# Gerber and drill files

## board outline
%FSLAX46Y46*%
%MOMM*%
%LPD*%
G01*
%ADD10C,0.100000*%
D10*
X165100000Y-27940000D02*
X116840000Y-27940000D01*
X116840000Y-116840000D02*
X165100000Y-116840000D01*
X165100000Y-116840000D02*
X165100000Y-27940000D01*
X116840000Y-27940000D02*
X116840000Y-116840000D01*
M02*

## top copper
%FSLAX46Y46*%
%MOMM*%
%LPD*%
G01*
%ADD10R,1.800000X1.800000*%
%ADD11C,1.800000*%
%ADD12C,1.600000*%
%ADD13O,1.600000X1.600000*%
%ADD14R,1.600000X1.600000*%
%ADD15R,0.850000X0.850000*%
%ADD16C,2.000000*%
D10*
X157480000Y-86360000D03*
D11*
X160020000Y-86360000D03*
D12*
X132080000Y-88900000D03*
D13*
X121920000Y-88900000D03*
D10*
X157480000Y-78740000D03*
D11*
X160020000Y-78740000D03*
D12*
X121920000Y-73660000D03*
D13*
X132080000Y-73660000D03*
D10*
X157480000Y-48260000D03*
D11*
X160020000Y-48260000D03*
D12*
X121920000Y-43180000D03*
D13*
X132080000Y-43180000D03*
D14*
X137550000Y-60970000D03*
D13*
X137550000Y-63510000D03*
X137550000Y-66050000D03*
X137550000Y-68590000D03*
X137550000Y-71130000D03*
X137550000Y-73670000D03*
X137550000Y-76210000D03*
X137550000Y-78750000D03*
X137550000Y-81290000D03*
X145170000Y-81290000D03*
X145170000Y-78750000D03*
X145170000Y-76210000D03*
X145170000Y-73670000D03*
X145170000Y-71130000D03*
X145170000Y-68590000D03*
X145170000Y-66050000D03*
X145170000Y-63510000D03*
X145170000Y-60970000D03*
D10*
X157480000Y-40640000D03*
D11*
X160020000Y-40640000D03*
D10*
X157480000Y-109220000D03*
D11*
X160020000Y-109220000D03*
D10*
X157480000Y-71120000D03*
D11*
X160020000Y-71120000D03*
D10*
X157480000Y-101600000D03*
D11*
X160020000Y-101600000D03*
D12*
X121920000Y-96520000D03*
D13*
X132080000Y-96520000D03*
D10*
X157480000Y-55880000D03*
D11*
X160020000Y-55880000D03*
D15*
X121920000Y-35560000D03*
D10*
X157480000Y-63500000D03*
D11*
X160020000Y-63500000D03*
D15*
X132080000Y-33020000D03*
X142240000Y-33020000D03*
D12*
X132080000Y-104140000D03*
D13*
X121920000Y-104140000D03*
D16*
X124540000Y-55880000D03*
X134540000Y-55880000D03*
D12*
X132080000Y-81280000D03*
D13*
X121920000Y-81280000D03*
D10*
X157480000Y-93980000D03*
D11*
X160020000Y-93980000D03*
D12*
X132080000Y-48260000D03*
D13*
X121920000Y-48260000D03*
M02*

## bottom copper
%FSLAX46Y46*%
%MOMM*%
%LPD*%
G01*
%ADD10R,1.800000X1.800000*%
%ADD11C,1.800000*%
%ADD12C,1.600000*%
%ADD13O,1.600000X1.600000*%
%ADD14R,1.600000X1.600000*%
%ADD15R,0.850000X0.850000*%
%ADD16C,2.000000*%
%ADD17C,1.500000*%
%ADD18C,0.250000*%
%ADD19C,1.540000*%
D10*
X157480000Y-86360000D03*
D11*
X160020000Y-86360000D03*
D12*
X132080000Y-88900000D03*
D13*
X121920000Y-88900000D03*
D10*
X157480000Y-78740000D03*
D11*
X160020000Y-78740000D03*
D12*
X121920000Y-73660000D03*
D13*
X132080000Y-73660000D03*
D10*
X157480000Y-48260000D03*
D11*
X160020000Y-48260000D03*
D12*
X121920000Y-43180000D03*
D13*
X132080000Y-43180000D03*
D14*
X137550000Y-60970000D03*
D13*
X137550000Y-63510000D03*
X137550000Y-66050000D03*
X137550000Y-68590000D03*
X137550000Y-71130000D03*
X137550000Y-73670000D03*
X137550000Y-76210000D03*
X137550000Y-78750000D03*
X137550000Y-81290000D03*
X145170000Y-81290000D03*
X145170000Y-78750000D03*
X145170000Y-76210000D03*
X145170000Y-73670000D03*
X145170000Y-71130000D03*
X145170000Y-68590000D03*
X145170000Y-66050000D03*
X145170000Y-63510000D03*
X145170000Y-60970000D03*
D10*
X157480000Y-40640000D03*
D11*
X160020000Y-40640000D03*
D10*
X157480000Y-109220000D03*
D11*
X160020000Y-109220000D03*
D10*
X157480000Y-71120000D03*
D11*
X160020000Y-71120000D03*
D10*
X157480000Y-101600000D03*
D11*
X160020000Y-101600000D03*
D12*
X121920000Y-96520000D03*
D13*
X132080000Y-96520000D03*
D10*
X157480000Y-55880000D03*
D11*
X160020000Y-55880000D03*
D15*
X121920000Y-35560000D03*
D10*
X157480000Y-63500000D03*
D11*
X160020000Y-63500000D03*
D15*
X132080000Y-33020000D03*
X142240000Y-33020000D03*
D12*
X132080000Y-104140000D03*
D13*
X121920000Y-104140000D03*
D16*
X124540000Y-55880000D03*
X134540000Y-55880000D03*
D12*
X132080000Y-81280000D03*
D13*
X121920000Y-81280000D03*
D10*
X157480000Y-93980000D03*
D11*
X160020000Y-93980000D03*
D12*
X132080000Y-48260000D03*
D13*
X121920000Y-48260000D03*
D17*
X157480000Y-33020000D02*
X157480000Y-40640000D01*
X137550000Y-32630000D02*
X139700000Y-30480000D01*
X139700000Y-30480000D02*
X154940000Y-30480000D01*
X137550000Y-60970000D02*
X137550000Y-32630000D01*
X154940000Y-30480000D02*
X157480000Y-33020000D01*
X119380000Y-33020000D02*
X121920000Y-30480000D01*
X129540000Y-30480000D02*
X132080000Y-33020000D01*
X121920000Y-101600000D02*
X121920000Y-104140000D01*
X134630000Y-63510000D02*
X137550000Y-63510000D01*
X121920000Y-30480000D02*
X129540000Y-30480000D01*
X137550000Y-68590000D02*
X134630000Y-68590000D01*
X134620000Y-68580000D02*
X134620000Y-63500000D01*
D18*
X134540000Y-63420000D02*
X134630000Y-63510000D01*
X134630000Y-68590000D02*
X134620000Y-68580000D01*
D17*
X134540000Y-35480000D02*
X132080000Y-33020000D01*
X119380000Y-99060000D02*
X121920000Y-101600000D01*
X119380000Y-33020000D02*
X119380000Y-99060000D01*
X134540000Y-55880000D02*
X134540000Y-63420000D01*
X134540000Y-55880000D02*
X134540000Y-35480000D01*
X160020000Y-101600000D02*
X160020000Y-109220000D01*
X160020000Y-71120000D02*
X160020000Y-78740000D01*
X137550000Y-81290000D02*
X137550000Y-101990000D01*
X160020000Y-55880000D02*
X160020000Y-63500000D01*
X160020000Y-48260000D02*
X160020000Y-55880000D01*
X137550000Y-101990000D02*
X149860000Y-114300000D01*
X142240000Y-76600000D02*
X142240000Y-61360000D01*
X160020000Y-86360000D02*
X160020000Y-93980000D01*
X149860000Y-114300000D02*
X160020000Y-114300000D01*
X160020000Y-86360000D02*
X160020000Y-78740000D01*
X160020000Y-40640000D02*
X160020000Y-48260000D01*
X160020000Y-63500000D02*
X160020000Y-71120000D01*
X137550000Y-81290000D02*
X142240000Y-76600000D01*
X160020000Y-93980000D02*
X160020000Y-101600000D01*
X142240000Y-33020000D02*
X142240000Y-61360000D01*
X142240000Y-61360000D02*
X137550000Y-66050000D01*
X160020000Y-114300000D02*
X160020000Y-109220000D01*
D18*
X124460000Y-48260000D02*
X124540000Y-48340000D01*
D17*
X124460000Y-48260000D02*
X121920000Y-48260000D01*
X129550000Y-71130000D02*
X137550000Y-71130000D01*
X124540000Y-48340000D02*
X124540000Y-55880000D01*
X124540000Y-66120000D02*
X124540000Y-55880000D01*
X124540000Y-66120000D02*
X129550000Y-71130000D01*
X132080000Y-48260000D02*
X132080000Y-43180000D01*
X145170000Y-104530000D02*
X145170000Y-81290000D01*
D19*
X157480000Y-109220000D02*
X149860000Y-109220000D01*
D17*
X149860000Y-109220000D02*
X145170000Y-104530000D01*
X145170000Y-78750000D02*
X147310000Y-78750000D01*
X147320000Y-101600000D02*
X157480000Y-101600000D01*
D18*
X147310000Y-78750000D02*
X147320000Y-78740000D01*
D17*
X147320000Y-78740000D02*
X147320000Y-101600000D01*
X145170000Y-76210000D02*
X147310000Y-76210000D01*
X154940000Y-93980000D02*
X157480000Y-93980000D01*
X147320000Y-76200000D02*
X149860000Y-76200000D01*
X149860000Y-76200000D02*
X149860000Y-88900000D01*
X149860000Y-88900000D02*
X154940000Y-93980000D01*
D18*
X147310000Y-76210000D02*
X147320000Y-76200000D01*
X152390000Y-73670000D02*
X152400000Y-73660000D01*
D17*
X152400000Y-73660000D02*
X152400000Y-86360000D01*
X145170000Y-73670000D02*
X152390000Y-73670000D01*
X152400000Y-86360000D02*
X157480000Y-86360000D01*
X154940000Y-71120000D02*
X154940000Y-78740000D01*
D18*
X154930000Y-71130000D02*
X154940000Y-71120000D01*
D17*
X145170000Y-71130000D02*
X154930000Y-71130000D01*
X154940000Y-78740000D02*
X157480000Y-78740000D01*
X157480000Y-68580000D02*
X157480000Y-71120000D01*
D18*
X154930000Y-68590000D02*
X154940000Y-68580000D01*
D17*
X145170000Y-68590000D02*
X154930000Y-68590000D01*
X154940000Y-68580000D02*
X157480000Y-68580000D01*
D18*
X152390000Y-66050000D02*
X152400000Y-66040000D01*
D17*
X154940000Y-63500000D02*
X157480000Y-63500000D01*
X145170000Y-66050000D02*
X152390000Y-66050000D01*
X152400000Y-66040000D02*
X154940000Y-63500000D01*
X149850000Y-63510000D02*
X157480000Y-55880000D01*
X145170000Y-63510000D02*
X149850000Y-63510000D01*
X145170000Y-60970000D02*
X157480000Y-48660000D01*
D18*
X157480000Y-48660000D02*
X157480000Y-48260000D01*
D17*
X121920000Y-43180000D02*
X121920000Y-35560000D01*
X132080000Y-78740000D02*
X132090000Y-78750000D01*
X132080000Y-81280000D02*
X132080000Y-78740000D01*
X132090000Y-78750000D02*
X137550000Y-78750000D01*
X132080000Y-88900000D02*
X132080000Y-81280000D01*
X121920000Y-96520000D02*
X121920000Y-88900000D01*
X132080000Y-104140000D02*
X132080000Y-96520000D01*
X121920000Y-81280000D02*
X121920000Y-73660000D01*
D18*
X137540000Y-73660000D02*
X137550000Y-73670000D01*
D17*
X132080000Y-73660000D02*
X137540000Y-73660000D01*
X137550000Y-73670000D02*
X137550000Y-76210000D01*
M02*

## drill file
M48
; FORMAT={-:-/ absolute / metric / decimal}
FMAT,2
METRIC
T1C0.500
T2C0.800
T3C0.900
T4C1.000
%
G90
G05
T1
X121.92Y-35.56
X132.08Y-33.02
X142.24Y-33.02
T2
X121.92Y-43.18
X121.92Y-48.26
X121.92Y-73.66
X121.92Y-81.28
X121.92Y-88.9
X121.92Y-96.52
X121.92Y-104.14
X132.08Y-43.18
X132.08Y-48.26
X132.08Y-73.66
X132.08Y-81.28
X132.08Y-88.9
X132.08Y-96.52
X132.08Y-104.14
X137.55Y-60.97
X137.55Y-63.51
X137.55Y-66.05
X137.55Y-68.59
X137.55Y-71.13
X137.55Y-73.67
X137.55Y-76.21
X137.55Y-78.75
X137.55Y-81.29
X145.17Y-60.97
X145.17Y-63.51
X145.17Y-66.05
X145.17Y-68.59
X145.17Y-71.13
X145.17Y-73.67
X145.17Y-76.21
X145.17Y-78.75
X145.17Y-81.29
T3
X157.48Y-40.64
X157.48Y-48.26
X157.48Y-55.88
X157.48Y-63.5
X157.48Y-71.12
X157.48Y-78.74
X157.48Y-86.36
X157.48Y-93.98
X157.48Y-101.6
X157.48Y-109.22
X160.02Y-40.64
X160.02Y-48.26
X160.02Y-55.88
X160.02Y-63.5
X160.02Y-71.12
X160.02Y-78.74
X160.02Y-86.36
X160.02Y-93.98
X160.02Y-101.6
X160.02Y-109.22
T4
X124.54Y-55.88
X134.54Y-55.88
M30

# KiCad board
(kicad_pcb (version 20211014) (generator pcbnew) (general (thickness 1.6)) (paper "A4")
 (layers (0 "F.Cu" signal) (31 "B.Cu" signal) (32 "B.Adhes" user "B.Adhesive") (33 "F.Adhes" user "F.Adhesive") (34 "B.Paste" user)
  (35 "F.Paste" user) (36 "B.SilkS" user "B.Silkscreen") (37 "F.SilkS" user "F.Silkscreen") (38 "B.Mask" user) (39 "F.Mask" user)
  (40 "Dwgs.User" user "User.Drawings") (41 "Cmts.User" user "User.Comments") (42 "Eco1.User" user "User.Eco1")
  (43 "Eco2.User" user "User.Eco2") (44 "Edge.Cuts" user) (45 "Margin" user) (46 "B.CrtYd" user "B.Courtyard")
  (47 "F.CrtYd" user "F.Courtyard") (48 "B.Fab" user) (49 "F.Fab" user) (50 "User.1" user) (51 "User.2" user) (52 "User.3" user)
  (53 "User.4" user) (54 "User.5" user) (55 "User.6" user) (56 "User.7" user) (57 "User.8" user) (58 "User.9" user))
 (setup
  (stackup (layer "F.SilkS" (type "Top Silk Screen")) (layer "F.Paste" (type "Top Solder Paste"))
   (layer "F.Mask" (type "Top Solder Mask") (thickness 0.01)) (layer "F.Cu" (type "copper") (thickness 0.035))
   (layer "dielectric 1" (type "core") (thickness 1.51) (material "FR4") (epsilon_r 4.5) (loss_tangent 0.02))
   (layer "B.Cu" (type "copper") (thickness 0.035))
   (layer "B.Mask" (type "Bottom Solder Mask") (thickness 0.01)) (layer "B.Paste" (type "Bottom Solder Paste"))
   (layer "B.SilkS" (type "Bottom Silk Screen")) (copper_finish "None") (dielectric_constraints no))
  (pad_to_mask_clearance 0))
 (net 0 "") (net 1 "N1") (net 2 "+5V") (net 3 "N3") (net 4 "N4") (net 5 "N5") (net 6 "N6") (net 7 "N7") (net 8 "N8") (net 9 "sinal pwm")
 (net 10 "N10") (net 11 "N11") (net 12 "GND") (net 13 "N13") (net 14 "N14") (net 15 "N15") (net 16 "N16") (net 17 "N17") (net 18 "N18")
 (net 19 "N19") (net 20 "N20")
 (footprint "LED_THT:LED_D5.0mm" (layer "F.Cu") (at 157.48 86.36)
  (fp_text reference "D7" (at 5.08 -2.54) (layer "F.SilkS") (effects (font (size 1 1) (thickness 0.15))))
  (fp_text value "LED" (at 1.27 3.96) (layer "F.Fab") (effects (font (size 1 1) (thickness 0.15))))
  (pad "1" thru_hole rect (at 0 0) (size 1.8 1.8) (drill 0.9) (layers *.Cu *.Mask) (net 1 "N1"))
  (pad "2" thru_hole circle (at 2.54 0) (size 1.8 1.8) (drill 0.9) (layers *.Cu *.Mask) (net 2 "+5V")))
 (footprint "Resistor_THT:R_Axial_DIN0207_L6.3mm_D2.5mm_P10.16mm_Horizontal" (layer "F.Cu") (at 132.08 88.9 180)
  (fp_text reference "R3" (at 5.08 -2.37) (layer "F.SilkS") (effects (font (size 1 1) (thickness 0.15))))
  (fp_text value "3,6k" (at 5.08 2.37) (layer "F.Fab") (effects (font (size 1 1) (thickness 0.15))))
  (pad "1" thru_hole circle (at 0 0 180) (size 1.6 1.6) (drill 0.8) (layers *.Cu *.Mask) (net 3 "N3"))
  (pad "2" thru_hole oval (at 10.16 0 180) (size 1.6 1.6) (drill 0.8) (layers *.Cu *.Mask) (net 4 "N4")))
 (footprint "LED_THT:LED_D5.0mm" (layer "F.Cu") (at 157.48 78.74)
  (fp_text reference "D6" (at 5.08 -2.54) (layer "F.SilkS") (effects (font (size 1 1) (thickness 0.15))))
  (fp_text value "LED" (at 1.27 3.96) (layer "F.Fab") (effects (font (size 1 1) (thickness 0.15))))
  (pad "1" thru_hole rect (at 0 0) (size 1.8 1.8) (drill 0.9) (layers *.Cu *.Mask) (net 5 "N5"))
  (pad "2" thru_hole circle (at 2.54 0) (size 1.8 1.8) (drill 0.9) (layers *.Cu *.Mask) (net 2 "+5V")))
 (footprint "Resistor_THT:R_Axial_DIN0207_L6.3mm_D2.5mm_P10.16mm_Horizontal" (layer "F.Cu") (at 121.92 73.66)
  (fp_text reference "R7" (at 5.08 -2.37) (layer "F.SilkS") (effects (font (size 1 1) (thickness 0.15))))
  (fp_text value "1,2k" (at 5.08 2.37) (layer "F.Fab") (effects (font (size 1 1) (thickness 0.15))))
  (pad "1" thru_hole circle (at 0 0) (size 1.6 1.6) (drill 0.8) (layers *.Cu *.Mask) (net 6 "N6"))
  (pad "2" thru_hole oval (at 10.16 0) (size 1.6 1.6) (drill 0.8) (layers *.Cu *.Mask) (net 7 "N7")))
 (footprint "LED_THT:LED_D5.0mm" (layer "F.Cu") (at 157.48 48.26)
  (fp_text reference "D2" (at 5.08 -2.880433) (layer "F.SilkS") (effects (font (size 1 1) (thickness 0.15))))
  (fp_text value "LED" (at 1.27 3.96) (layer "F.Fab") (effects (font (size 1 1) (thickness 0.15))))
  (pad "1" thru_hole rect (at 0 0) (size 1.8 1.8) (drill 0.9) (layers *.Cu *.Mask) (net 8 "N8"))
  (pad "2" thru_hole circle (at 2.54 0) (size 1.8 1.8) (drill 0.9) (layers *.Cu *.Mask) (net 2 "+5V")))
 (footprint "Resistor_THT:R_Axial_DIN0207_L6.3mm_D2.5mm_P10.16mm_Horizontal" (layer "F.Cu") (at 121.92 43.18)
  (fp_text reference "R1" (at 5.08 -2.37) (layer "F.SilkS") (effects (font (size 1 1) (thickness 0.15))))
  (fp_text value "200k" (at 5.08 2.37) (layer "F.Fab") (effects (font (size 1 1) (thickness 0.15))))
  (pad "1" thru_hole circle (at 0 0) (size 1.6 1.6) (drill 0.8) (layers *.Cu *.Mask) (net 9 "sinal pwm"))
  (pad "2" thru_hole oval (at 10.16 0) (size 1.6 1.6) (drill 0.8) (layers *.Cu *.Mask) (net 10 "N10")))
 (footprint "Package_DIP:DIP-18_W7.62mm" (layer "F.Cu") (at 137.55 60.97)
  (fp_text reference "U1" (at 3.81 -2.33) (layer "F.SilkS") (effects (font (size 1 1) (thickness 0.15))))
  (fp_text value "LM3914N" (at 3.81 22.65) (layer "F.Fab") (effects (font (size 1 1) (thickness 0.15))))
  (pad "1" thru_hole rect (at 0 0) (size 1.6 1.6) (drill 0.8) (layers *.Cu *.Mask) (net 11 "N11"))
  (pad "2" thru_hole oval (at 0 2.54) (size 1.6 1.6) (drill 0.8) (layers *.Cu *.Mask) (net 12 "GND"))
  (pad "3" thru_hole oval (at 0 5.08) (size 1.6 1.6) (drill 0.8) (layers *.Cu *.Mask) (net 2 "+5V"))
  (pad "4" thru_hole oval (at 0 7.62) (size 1.6 1.6) (drill 0.8) (layers *.Cu *.Mask) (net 12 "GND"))
  (pad "5" thru_hole oval (at 0 10.16) (size 1.6 1.6) (drill 0.8) (layers *.Cu *.Mask) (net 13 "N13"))
  (pad "6" thru_hole oval (at 0 12.7) (size 1.6 1.6) (drill 0.8) (layers *.Cu *.Mask) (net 7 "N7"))
  (pad "7" thru_hole oval (at 0 15.24) (size 1.6 1.6) (drill 0.8) (layers *.Cu *.Mask) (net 7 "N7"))
  (pad "8" thru_hole oval (at 0 17.78) (size 1.6 1.6) (drill 0.8) (layers *.Cu *.Mask) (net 3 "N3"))
  (pad "9" thru_hole oval (at 0 20.32) (size 1.6 1.6) (drill 0.8) (layers *.Cu *.Mask) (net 2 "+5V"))
  (pad "10" thru_hole oval (at 7.62 20.32) (size 1.6 1.6) (drill 0.8) (layers *.Cu *.Mask) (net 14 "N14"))
  (pad "11" thru_hole oval (at 7.62 17.78) (size 1.6 1.6) (drill 0.8) (layers *.Cu *.Mask) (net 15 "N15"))
  (pad "12" thru_hole oval (at 7.62 15.24) (size 1.6 1.6) (drill 0.8) (layers *.Cu *.Mask) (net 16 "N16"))
  (pad "13" thru_hole oval (at 7.62 12.7) (size 1.6 1.6) (drill 0.8) (layers *.Cu *.Mask) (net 1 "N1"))
  (pad "14" thru_hole oval (at 7.62 10.16) (size 1.6 1.6) (drill 0.8) (layers *.Cu *.Mask) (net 5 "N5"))
  (pad "15" thru_hole oval (at 7.62 7.62) (size 1.6 1.6) (drill 0.8) (layers *.Cu *.Mask) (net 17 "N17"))
  (pad "16" thru_hole oval (at 7.62 5.08) (size 1.6 1.6) (drill 0.8) (layers *.Cu *.Mask) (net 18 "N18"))
  (pad "17" thru_hole oval (at 7.62 2.54) (size 1.6 1.6) (drill 0.8) (layers *.Cu *.Mask) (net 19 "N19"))
  (pad "18" thru_hole oval (at 7.62 0) (size 1.6 1.6) (drill 0.8) (layers *.Cu *.Mask) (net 8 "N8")))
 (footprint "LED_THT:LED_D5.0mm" (layer "F.Cu") (at 157.48 40.64)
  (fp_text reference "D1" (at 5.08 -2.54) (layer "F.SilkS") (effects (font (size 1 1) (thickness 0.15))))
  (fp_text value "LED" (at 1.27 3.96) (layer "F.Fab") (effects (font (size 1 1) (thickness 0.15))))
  (pad "1" thru_hole rect (at 0 0) (size 1.8 1.8) (drill 0.9) (layers *.Cu *.Mask) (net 11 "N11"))
  (pad "2" thru_hole circle (at 2.54 0) (size 1.8 1.8) (drill 0.9) (layers *.Cu *.Mask) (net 2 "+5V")))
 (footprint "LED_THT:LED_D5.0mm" (layer "F.Cu") (at 157.48 109.22)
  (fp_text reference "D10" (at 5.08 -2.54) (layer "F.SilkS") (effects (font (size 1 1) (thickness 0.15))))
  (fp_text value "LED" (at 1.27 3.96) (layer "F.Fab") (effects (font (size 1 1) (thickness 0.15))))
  (pad "1" thru_hole rect (at 0 0) (size 1.8 1.8) (drill 0.9) (layers *.Cu *.Mask) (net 14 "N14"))
  (pad "2" thru_hole circle (at 2.54 0) (size 1.8 1.8) (drill 0.9) (layers *.Cu *.Mask) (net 2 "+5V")))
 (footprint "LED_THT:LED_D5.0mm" (layer "F.Cu") (at 157.48 71.12)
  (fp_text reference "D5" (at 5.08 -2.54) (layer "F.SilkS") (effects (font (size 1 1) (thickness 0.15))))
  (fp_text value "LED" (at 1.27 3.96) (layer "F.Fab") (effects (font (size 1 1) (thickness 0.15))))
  (pad "1" thru_hole rect (at 0 0) (size 1.8 1.8) (drill 0.9) (layers *.Cu *.Mask) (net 17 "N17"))
  (pad "2" thru_hole circle (at 2.54 0) (size 1.8 1.8) (drill 0.9) (layers *.Cu *.Mask) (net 2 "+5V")))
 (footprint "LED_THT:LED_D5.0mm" (layer "F.Cu") (at 157.48 101.6)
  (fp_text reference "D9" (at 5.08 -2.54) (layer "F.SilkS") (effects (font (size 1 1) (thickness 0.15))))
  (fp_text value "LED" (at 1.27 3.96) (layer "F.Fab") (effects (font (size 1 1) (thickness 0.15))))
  (pad "1" thru_hole rect (at 0 0) (size 1.8 1.8) (drill 0.9) (layers *.Cu *.Mask) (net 15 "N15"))
  (pad "2" thru_hole circle (at 2.54 0) (size 1.8 1.8) (drill 0.9) (layers *.Cu *.Mask) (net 2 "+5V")))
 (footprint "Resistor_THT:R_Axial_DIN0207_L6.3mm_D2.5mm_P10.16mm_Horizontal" (layer "F.Cu") (at 121.92 96.52)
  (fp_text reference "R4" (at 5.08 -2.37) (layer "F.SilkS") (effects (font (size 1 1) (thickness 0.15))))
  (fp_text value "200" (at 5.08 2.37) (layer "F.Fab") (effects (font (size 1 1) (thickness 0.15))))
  (pad "1" thru_hole circle (at 0 0) (size 1.6 1.6) (drill 0.8) (layers *.Cu *.Mask) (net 4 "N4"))
  (pad "2" thru_hole oval (at 10.16 0) (size 1.6 1.6) (drill 0.8) (layers *.Cu *.Mask) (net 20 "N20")))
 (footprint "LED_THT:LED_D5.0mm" (layer "F.Cu") (at 157.48 55.88)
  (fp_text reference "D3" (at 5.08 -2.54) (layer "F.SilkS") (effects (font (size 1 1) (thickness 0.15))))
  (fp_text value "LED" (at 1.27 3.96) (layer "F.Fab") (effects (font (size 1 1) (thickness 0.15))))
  (pad "1" thru_hole rect (at 0 0) (size 1.8 1.8) (drill 0.9) (layers *.Cu *.Mask) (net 19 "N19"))
  (pad "2" thru_hole circle (at 2.54 0) (size 1.8 1.8) (drill 0.9) (layers *.Cu *.Mask) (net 2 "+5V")))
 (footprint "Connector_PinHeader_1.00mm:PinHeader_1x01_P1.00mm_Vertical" (layer "F.Cu") (at 121.92 35.56)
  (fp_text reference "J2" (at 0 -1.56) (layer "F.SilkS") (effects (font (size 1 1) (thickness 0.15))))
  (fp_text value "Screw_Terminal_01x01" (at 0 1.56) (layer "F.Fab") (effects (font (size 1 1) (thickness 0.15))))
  (pad "1" thru_hole rect (at 0 0) (size 0.85 0.85) (drill 0.5) (layers *.Cu *.Mask) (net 9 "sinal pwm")))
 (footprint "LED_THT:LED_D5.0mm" (layer "F.Cu") (at 157.48 63.5)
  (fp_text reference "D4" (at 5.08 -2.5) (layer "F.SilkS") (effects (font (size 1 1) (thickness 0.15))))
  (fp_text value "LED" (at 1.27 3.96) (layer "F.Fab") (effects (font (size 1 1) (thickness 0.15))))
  (pad "1" thru_hole rect (at 0 0) (size 1.8 1.8) (drill 0.9) (layers *.Cu *.Mask) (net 18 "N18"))
  (pad "2" thru_hole circle (at 2.54 0) (size 1.8 1.8) (drill 0.9) (layers *.Cu *.Mask) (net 2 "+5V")))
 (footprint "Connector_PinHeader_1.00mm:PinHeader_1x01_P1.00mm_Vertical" (layer "F.Cu") (at 132.08 33.02)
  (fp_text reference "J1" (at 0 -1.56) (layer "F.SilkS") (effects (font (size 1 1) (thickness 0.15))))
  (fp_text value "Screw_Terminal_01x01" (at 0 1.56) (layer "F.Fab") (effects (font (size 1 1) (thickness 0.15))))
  (pad "1" thru_hole rect (at 0 0) (size 0.85 0.85) (drill 0.5) (layers *.Cu *.Mask) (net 12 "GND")))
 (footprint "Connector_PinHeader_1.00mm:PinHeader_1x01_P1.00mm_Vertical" (layer "F.Cu") (at 142.24 33.02)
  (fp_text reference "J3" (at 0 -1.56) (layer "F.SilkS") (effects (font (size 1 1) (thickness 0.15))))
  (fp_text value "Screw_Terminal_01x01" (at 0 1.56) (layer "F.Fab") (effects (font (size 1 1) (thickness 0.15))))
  (pad "1" thru_hole rect (at 0 0) (size 0.85 0.85) (drill 0.5) (layers *.Cu *.Mask) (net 2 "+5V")))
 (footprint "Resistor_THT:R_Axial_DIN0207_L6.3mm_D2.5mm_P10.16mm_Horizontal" (layer "F.Cu") (at 132.08 104.14 180)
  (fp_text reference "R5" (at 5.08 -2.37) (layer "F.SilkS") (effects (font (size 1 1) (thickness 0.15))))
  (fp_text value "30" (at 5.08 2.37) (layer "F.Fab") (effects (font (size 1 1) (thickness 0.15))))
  (pad "1" thru_hole circle (at 0 0 180) (size 1.6 1.6) (drill 0.8) (layers *.Cu *.Mask) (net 20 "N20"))
  (pad "2" thru_hole oval (at 10.16 0 180) (size 1.6 1.6) (drill 0.8) (layers *.Cu *.Mask) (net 12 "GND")))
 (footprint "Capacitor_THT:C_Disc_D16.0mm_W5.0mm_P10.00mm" (layer "F.Cu") (at 124.54 55.88)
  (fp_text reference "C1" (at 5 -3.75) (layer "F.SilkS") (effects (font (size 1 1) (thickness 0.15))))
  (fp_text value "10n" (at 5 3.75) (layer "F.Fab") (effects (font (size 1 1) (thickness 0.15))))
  (pad "1" thru_hole circle (at 0 0) (size 2 2) (drill 1) (layers *.Cu *.Mask) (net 13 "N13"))
  (pad "2" thru_hole circle (at 10 0) (size 2 2) (drill 1) (layers *.Cu *.Mask) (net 12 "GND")))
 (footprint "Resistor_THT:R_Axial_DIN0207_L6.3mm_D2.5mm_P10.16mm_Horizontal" (layer "F.Cu") (at 132.08 81.28 180)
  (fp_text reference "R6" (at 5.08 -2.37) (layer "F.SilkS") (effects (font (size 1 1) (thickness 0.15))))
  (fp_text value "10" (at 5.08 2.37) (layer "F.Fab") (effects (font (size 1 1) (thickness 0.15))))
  (pad "1" thru_hole circle (at 0 0 180) (size 1.6 1.6) (drill 0.8) (layers *.Cu *.Mask) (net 3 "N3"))
  (pad "2" thru_hole oval (at 10.16 0 180) (size 1.6 1.6) (drill 0.8) (layers *.Cu *.Mask) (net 6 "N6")))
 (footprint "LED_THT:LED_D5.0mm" (layer "F.Cu") (at 157.48 93.98)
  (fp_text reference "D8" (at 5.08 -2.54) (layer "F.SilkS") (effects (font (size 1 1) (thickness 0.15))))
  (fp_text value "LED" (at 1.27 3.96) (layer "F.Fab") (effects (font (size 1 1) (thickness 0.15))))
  (pad "1" thru_hole rect (at 0 0) (size 1.8 1.8) (drill 0.9) (layers *.Cu *.Mask) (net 16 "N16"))
  (pad "2" thru_hole circle (at 2.54 0) (size 1.8 1.8) (drill 0.9) (layers *.Cu *.Mask) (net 2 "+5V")))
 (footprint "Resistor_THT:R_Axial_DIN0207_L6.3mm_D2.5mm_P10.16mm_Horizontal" (layer "F.Cu") (at 132.08 48.26 180)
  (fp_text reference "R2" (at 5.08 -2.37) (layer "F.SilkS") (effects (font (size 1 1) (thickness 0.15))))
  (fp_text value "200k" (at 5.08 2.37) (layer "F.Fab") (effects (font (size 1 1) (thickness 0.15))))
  (pad "1" thru_hole circle (at 0 0 180) (size 1.6 1.6) (drill 0.8) (layers *.Cu *.Mask) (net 10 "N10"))
  (pad "2" thru_hole oval (at 10.16 0 180) (size 1.6 1.6) (drill 0.8) (layers *.Cu *.Mask) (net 13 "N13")))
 (gr_rect (start 177.8 134.62) (end 177.8 134.62) (layer "B.Cu") (width 0.2) (fill none))
 (gr_line (start 165.1 27.94) (end 116.84 27.94) (layer "Edge.Cuts") (width 0.1))
 (gr_line (start 116.84 116.84) (end 165.1 116.84) (layer "Edge.Cuts") (width 0.1))
 (gr_line (start 165.1 116.84) (end 165.1 27.94) (layer "Edge.Cuts") (width 0.1))
 (gr_line (start 116.84 27.94) (end 116.84 116.84) (layer "Edge.Cuts") (width 0.1))
 (segment (start 157.48 33.02) (end 157.48 40.64) (width 1.5) (layer "B.Cu") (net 11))
 (segment (start 137.55 32.63) (end 139.7 30.48) (width 1.5) (layer "B.Cu") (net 11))
 (segment (start 139.7 30.48) (end 154.94 30.48) (width 1.5) (layer "B.Cu") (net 11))
 (segment (start 137.55 60.97) (end 137.55 32.63) (width 1.5) (layer "B.Cu") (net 11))
 (segment (start 154.94 30.48) (end 157.48 33.02) (width 1.5) (layer "B.Cu") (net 11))
 (segment (start 119.38 33.02) (end 121.92 30.48) (width 1.5) (layer "B.Cu") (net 12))
 (segment (start 129.54 30.48) (end 132.08 33.02) (width 1.5) (layer "B.Cu") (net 12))
 (segment (start 121.92 101.6) (end 121.92 104.14) (width 1.5) (layer "B.Cu") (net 12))
 (segment (start 134.63 63.51) (end 137.55 63.51) (width 1.5) (layer "B.Cu") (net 12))
 (segment (start 121.92 30.48) (end 129.54 30.48) (width 1.5) (layer "B.Cu") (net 12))
 (segment (start 137.55 68.59) (end 134.63 68.59) (width 1.5) (layer "B.Cu") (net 12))
 (segment (start 134.62 68.58) (end 134.62 63.5) (width 1.5) (layer "B.Cu") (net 12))
 (segment (start 134.54 63.42) (end 134.63 63.51) (width 0.25) (layer "B.Cu") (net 12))
 (segment (start 134.63 68.59) (end 134.62 68.58) (width 0.25) (layer "B.Cu") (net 12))
 (segment (start 134.54 35.48) (end 132.08 33.02) (width 1.5) (layer "B.Cu") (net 12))
 (segment (start 119.38 99.06) (end 121.92 101.6) (width 1.5) (layer "B.Cu") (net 12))
 (segment (start 119.38 33.02) (end 119.38 99.06) (width 1.5) (layer "B.Cu") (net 12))
 (segment (start 134.54 55.88) (end 134.54 63.42) (width 1.5) (layer "B.Cu") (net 12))
 (segment (start 134.54 55.88) (end 134.54 35.48) (width 1.5) (layer "B.Cu") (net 12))
 (segment (start 160.02 101.6) (end 160.02 109.22) (width 1.5) (layer "B.Cu") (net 2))
 (segment (start 160.02 71.12) (end 160.02 78.74) (width 1.5) (layer "B.Cu") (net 2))
 (segment (start 137.55 81.29) (end 137.55 101.99) (width 1.5) (layer "B.Cu") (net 2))
 (segment (start 160.02 55.88) (end 160.02 63.5) (width 1.5) (layer "B.Cu") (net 2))
 (segment (start 160.02 48.26) (end 160.02 55.88) (width 1.5) (layer "B.Cu") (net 2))
 (segment (start 137.55 101.99) (end 149.86 114.3) (width 1.5) (layer "B.Cu") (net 2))
 (segment (start 142.24 76.6) (end 142.24 61.36) (width 1.5) (layer "B.Cu") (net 2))
 (segment (start 160.02 86.36) (end 160.02 93.98) (width 1.5) (layer "B.Cu") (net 2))
 (segment (start 149.86 114.3) (end 160.02 114.3) (width 1.5) (layer "B.Cu") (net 2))
 (segment (start 160.02 86.36) (end 160.02 78.74) (width 1.5) (layer "B.Cu") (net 2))
 (segment (start 160.02 40.64) (end 160.02 48.26) (width 1.5) (layer "B.Cu") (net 2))
 (segment (start 160.02 63.5) (end 160.02 71.12) (width 1.5) (layer "B.Cu") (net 2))
 (segment (start 137.55 81.29) (end 142.24 76.6) (width 1.5) (layer "B.Cu") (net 2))
 (segment (start 160.02 93.98) (end 160.02 101.6) (width 1.5) (layer "B.Cu") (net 2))
 (segment (start 142.24 33.02) (end 142.24 61.36) (width 1.5) (layer "B.Cu") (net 2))
 (segment (start 142.24 61.36) (end 137.55 66.05) (width 1.5) (layer "B.Cu") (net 2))
 (segment (start 160.02 114.3) (end 160.02 109.22) (width 1.5) (layer "B.Cu") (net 2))
 (segment (start 124.46 48.26) (end 124.54 48.34) (width 0.25) (layer "B.Cu") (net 13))
 (segment (start 124.46 48.26) (end 121.92 48.26) (width 1.5) (layer "B.Cu") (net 13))
 (segment (start 129.55 71.13) (end 137.55 71.13) (width 1.5) (layer "B.Cu") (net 13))
 (segment (start 124.54 48.34) (end 124.54 55.88) (width 1.5) (layer "B.Cu") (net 13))
 (segment (start 124.54 66.12) (end 124.54 55.88) (width 1.5) (layer "B.Cu") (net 13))
 (segment (start 124.54 66.12) (end 129.55 71.13) (width 1.5) (layer "B.Cu") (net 13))
 (segment (start 132.08 48.26) (end 132.08 43.18) (width 1.5) (layer "B.Cu") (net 10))
 (segment (start 145.17 104.53) (end 145.17 81.29) (width 1.5) (layer "B.Cu") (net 14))
 (segment (start 157.48 109.22) (end 149.86 109.22) (width 1.54) (layer "B.Cu") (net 14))
 (segment (start 149.86 109.22) (end 145.17 104.53) (width 1.5) (layer "B.Cu") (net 14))
 (segment (start 145.17 78.75) (end 147.31 78.75) (width 1.5) (layer "B.Cu") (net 15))
 (segment (start 147.32 101.6) (end 157.48 101.6) (width 1.5) (layer "B.Cu") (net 15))
 (segment (start 147.31 78.75) (end 147.32 78.74) (width 0.25) (layer "B.Cu") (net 15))
 (segment (start 147.32 78.74) (end 147.32 101.6) (width 1.5) (layer "B.Cu") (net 15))
 (segment (start 145.17 76.21) (end 147.31 76.21) (width 1.5) (layer "B.Cu") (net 16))
 (segment (start 154.94 93.98) (end 157.48 93.98) (width 1.5) (layer "B.Cu") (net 16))
 (segment (start 147.32 76.2) (end 149.86 76.2) (width 1.5) (layer "B.Cu") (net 16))
 (segment (start 149.86 76.2) (end 149.86 88.9) (width 1.5) (layer "B.Cu") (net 16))
 (segment (start 149.86 88.9) (end 154.94 93.98) (width 1.5) (layer "B.Cu") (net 16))
 (segment (start 147.31 76.21) (end 147.32 76.2) (width 0.25) (layer "B.Cu") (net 16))
 (segment (start 152.39 73.67) (end 152.4 73.66) (width 0.25) (layer "B.Cu") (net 1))
 (segment (start 152.4 73.66) (end 152.4 86.36) (width 1.5) (layer "B.Cu") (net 1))
 (segment (start 145.17 73.67) (end 152.39 73.67) (width 1.5) (layer "B.Cu") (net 1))
 (segment (start 152.4 86.36) (end 157.48 86.36) (width 1.5) (layer "B.Cu") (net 1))
 (segment (start 154.94 71.12) (end 154.94 78.74) (width 1.5) (layer "B.Cu") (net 5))
 (segment (start 154.93 71.13) (end 154.94 71.12) (width 0.25) (layer "B.Cu") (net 5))
 (segment (start 145.17 71.13) (end 154.93 71.13) (width 1.5) (layer "B.Cu") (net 5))
 (segment (start 154.94 78.74) (end 157.48 78.74) (width 1.5) (layer "B.Cu") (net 5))
 (segment (start 157.48 68.58) (end 157.48 71.12) (width 1.5) (layer "B.Cu") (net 17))
 (segment (start 154.93 68.59) (end 154.94 68.58) (width 0.25) (layer "B.Cu") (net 17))
 (segment (start 145.17 68.59) (end 154.93 68.59) (width 1.5) (layer "B.Cu") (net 17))
 (segment (start 154.94 68.58) (end 157.48 68.58) (width 1.5) (layer "B.Cu") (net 17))
 (segment (start 152.39 66.05) (end 152.4 66.04) (width 0.25) (layer "B.Cu") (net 18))
 (segment (start 154.94 63.5) (end 157.48 63.5) (width 1.5) (layer "B.Cu") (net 18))
 (segment (start 145.17 66.05) (end 152.39 66.05) (width 1.5) (layer "B.Cu") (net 18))
 (segment (start 152.4 66.04) (end 154.94 63.5) (width 1.5) (layer "B.Cu") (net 18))
 (segment (start 149.85 63.51) (end 157.48 55.88) (width 1.5) (layer "B.Cu") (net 19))
 (segment (start 145.17 63.51) (end 149.85 63.51) (width 1.5) (layer "B.Cu") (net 19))
 (segment (start 145.17 60.97) (end 157.48 48.66) (width 1.5) (layer "B.Cu") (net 8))
 (segment (start 157.48 48.66) (end 157.48 48.26) (width 0.25) (layer "B.Cu") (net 8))
 (segment (start 121.92 43.18) (end 121.92 35.56) (width 1.5) (layer "B.Cu") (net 9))
 (segment (start 132.08 78.74) (end 132.09 78.75) (width 1.5) (layer "B.Cu") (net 3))
 (segment (start 132.08 81.28) (end 132.08 78.74) (width 1.5) (layer "B.Cu") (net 3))
 (segment (start 132.09 78.75) (end 137.55 78.75) (width 1.5) (layer "B.Cu") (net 3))
 (segment (start 132.08 88.9) (end 132.08 81.28) (width 1.5) (layer "B.Cu") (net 3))
 (segment (start 121.92 96.52) (end 121.92 88.9) (width 1.5) (layer "B.Cu") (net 4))
 (segment (start 132.08 104.14) (end 132.08 96.52) (width 1.5) (layer "B.Cu") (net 20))
 (segment (start 121.92 81.28) (end 121.92 73.66) (width 1.5) (layer "B.Cu") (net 6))
 (segment (start 137.54 73.66) (end 137.55 73.67) (width 0.25) (layer "B.Cu") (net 7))
 (segment (start 132.08 73.66) (end 137.54 73.66) (width 1.5) (layer "B.Cu") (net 7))
 (segment (start 137.55 73.67) (end 137.55 76.21) (width 1.5) (layer "B.Cu") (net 7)))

